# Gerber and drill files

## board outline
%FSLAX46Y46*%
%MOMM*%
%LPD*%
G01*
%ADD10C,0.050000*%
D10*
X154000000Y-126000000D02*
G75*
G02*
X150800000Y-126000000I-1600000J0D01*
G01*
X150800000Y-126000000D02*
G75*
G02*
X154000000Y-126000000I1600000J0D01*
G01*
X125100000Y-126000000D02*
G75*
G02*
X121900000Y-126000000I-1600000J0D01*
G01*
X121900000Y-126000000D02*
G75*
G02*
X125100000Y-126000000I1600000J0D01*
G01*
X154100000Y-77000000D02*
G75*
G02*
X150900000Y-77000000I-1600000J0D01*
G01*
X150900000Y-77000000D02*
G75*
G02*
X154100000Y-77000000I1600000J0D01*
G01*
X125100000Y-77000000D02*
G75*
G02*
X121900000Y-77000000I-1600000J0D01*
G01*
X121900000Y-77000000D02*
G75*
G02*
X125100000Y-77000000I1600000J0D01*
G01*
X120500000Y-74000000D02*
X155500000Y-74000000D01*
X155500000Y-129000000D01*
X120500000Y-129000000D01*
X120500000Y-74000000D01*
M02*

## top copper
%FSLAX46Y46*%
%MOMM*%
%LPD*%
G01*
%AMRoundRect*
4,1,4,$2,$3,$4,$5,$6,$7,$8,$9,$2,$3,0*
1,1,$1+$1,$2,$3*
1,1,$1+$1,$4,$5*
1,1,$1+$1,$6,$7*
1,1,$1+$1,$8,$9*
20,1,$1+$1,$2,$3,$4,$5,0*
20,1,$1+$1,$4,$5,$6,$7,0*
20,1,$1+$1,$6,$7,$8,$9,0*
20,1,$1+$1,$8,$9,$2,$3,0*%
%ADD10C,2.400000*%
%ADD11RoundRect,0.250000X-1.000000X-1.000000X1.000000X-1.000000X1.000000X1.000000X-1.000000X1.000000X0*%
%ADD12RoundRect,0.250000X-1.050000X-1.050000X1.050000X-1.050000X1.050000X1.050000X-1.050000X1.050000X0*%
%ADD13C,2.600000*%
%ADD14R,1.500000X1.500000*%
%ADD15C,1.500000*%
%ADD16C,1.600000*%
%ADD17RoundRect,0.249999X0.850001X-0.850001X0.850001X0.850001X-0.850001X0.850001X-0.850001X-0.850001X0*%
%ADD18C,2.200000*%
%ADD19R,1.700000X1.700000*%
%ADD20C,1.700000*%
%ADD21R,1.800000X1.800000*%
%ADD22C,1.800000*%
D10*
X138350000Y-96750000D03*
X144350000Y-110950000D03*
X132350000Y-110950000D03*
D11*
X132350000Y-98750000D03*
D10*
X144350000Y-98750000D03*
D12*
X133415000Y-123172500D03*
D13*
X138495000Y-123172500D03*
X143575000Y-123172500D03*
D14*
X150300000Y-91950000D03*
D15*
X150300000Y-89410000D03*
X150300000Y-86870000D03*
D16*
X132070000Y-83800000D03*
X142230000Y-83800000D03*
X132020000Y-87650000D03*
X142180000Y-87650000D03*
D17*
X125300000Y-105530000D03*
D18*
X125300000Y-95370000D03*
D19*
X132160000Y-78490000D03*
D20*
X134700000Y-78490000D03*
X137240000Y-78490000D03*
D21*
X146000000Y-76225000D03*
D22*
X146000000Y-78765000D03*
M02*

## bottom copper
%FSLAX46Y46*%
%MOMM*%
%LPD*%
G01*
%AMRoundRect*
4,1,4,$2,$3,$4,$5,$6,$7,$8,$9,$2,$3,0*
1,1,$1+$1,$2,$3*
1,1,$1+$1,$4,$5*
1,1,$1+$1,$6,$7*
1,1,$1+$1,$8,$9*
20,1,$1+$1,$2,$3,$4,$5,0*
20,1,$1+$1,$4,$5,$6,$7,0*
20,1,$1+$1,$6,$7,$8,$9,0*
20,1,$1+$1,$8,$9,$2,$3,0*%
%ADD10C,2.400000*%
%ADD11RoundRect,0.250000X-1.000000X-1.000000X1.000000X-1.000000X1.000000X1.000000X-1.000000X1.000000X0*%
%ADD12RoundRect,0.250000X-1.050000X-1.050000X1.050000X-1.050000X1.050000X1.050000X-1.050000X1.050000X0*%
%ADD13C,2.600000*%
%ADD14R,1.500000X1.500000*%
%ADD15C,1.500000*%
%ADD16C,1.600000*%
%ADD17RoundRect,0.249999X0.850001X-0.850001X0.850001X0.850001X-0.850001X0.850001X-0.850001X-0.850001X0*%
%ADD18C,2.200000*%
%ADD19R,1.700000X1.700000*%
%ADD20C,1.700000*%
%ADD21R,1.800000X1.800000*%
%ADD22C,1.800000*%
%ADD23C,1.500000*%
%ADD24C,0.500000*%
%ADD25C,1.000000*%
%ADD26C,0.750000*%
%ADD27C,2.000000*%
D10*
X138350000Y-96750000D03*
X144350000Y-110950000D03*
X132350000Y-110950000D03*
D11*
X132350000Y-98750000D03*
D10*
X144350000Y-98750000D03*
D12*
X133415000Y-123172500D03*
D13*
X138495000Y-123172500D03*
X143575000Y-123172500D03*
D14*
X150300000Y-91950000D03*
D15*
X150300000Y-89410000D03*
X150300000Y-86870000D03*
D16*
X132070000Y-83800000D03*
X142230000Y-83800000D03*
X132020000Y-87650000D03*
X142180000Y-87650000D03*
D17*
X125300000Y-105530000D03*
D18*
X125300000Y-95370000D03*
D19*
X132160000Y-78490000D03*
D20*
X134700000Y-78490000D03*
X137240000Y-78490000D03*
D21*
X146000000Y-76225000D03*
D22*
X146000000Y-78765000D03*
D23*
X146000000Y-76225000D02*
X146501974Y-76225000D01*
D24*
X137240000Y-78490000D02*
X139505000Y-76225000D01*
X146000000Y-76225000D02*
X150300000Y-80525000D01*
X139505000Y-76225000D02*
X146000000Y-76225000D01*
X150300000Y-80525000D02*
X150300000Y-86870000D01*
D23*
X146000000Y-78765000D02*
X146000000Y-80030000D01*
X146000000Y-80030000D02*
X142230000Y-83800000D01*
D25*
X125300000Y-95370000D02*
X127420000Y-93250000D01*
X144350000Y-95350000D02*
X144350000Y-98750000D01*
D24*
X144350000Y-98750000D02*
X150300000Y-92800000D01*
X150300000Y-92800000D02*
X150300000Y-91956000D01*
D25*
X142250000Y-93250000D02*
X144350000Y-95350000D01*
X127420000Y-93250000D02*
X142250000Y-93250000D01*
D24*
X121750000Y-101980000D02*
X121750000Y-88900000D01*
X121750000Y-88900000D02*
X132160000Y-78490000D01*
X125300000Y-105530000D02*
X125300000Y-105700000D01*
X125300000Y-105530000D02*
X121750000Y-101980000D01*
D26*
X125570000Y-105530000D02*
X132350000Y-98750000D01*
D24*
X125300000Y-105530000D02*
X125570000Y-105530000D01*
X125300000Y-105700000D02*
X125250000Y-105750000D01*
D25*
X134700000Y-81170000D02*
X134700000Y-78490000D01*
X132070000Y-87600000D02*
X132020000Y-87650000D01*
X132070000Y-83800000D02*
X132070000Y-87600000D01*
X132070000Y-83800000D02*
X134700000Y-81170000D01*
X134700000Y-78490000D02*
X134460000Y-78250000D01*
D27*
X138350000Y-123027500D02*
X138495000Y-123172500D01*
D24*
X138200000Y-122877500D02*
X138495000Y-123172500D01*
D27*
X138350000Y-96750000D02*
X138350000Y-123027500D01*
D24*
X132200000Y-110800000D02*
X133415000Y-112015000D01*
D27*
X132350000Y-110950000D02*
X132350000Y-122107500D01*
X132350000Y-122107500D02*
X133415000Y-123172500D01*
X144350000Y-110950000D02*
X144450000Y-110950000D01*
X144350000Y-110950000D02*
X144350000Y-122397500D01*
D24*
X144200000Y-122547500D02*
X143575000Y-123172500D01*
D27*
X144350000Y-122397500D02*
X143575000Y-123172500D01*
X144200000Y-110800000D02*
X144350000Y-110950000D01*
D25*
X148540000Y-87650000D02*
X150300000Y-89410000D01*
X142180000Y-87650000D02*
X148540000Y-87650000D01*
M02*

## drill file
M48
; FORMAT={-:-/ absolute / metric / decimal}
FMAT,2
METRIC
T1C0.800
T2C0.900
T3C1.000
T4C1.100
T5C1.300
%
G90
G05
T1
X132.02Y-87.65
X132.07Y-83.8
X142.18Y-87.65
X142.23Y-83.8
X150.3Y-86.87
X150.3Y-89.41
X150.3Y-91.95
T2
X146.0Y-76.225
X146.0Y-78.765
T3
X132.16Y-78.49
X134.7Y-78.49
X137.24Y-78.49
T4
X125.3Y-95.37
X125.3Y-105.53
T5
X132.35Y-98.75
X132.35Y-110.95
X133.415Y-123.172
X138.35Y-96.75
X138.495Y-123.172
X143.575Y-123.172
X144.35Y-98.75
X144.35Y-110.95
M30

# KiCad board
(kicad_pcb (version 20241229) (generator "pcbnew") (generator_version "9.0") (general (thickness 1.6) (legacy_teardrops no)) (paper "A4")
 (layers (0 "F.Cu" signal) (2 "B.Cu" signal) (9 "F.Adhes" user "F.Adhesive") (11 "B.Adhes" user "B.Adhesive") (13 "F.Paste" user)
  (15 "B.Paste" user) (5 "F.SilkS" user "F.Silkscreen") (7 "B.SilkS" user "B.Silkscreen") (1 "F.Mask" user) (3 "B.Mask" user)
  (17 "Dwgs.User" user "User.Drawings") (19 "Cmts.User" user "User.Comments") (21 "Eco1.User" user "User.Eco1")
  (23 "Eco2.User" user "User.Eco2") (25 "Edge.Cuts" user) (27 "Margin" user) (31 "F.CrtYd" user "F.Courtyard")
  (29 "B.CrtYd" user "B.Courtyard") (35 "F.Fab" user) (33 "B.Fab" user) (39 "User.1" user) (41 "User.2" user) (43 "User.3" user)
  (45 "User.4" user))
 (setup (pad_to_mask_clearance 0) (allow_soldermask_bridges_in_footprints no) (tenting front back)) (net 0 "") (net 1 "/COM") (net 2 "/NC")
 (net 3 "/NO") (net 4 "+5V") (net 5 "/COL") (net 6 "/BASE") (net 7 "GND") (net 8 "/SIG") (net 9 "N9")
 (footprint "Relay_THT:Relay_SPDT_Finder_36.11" (layer "F.Cu") (at 132.35 98.75)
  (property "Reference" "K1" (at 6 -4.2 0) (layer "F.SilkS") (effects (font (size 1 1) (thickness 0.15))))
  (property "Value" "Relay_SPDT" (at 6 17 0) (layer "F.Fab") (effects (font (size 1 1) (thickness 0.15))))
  (pad "11" thru_hole circle (at 6 -2) (size 2.4 2.4) (drill 1.3) (layers "*.Cu" "*.Mask") (remove_unused_layers no) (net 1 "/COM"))
  (pad "12" thru_hole circle (at 12 12.2) (size 2.4 2.4) (drill 1.3) (layers "*.Cu" "*.Mask") (remove_unused_layers no) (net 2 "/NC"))
  (pad "14" thru_hole circle (at 0 12.2) (size 2.4 2.4) (drill 1.3) (layers "*.Cu" "*.Mask") (remove_unused_layers no) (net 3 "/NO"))
  (pad "A1" thru_hole roundrect (at 0 0) (size 2.5 2.5) (drill 1.3) (layers "*.Cu" "*.Mask") (remove_unused_layers no)
   (roundrect_rratio 0.1) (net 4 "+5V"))
  (pad "A2" thru_hole circle (at 12 0) (size 2.4 2.4) (drill 1.3) (layers "*.Cu" "*.Mask") (remove_unused_layers no) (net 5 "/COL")))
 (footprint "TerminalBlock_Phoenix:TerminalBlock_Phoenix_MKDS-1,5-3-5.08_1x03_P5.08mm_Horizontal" (layer "F.Cu") (at 133.415 123.1725)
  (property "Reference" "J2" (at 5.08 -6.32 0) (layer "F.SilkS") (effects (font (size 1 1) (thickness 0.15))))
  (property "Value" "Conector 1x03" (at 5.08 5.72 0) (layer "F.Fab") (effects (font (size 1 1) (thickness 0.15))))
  (pad "1" thru_hole roundrect (at 0 0) (size 2.6 2.6) (drill 1.3) (layers "*.Cu" "*.Mask") (remove_unused_layers no)
   (roundrect_rratio 0.096154) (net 3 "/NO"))
  (pad "2" thru_hole circle (at 5.08 0) (size 2.6 2.6) (drill 1.3) (layers "*.Cu" "*.Mask") (remove_unused_layers no) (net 1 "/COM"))
  (pad "3" thru_hole circle (at 10.16 0) (size 2.6 2.6) (drill 1.3) (layers "*.Cu" "*.Mask") (remove_unused_layers no) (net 2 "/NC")))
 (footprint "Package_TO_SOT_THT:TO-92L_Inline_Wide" (layer "F.Cu") (at 150.3 91.95 90)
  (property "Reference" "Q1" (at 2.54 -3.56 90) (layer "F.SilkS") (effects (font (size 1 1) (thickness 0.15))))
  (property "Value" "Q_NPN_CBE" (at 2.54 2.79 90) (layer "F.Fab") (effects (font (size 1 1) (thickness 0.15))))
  (pad "1" thru_hole rect (at 0 0 90) (size 1.5 1.5) (drill 0.8) (layers "*.Cu" "*.Mask") (remove_unused_layers no) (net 5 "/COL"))
  (pad "2" thru_hole circle (at 2.54 0 90) (size 1.5 1.5) (drill 0.8) (layers "*.Cu" "*.Mask") (remove_unused_layers no) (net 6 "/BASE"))
  (pad "3" thru_hole circle (at 5.08 0 90) (size 1.5 1.5) (drill 0.8) (layers "*.Cu" "*.Mask") (remove_unused_layers no) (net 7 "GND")))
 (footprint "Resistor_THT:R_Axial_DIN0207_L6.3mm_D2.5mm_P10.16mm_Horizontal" (layer "F.Cu") (at 132.07 83.8)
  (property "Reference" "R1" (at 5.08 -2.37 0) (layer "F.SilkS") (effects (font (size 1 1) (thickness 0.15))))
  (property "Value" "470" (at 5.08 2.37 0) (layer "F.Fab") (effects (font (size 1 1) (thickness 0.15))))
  (pad "1" thru_hole circle (at 0 0) (size 1.6 1.6) (drill 0.8) (layers "*.Cu" "*.Mask") (remove_unused_layers no) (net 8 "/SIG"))
  (pad "2" thru_hole circle (at 10.16 0) (size 1.6 1.6) (drill 0.8) (layers "*.Cu" "*.Mask") (remove_unused_layers no) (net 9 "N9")))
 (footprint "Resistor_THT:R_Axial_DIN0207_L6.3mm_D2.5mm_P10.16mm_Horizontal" (layer "F.Cu") (at 132.02 87.65)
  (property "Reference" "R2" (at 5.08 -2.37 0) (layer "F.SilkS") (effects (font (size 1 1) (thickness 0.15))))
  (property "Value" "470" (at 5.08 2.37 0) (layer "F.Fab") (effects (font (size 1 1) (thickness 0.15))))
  (pad "1" thru_hole circle (at 0 0) (size 1.6 1.6) (drill 0.8) (layers "*.Cu" "*.Mask") (remove_unused_layers no) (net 8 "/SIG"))
  (pad "2" thru_hole circle (at 10.16 0) (size 1.6 1.6) (drill 0.8) (layers "*.Cu" "*.Mask") (remove_unused_layers no) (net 6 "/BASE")))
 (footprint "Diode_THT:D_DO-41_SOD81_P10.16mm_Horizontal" (layer "F.Cu") (at 125.3 105.53 90)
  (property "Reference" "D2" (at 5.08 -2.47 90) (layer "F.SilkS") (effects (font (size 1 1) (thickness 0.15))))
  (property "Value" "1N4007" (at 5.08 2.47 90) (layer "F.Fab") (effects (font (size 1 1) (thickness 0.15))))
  (pad "1" thru_hole roundrect (at 0 0 90) (size 2.2 2.2) (drill 1.1) (layers "*.Cu" "*.Mask") (remove_unused_layers no)
   (roundrect_rratio 0.113636) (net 4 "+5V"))
  (pad "2" thru_hole circle (at 10.16 0 90) (size 2.2 2.2) (drill 1.1) (layers "*.Cu" "*.Mask") (remove_unused_layers no) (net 5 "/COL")))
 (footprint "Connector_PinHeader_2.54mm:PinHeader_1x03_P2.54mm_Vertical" (layer "F.Cu") (at 132.16 78.49 90)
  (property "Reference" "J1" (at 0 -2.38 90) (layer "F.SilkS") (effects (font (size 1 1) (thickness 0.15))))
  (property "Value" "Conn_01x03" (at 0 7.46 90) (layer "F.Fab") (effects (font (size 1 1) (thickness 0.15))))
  (pad "1" thru_hole rect (at 0 0 90) (size 1.7 1.7) (drill 1) (layers "*.Cu" "*.Mask") (remove_unused_layers no) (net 4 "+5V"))
  (pad "2" thru_hole circle (at 0 2.54 90) (size 1.7 1.7) (drill 1) (layers "*.Cu" "*.Mask") (remove_unused_layers no) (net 8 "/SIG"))
  (pad "3" thru_hole circle (at 0 5.08 90) (size 1.7 1.7) (drill 1) (layers "*.Cu" "*.Mask") (remove_unused_layers no) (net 7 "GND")))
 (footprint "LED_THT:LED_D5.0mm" (layer "F.Cu") (at 146 76.225 -90)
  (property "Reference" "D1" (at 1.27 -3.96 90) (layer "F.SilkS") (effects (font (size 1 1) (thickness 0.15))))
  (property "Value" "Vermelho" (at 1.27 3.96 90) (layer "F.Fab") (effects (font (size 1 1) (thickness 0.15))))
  (pad "1" thru_hole rect (at 0 0 270) (size 1.8 1.8) (drill 0.9) (layers "*.Cu" "*.Mask") (remove_unused_layers no) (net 7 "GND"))
  (pad "2" thru_hole circle (at 2.54 0 270) (size 1.8 1.8) (drill 0.9) (layers "*.Cu" "*.Mask") (remove_unused_layers no) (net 9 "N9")))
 (gr_circle (center 152.4 126) (end 154 126) (stroke (width 0.05) (type solid)) (fill no) (layer "Edge.Cuts"))
 (gr_circle (center 123.5 126) (end 125.1 126) (stroke (width 0.05) (type solid)) (fill no) (layer "Edge.Cuts"))
 (gr_circle (center 152.5 77) (end 154.1 77) (stroke (width 0.05) (type solid)) (fill no) (layer "Edge.Cuts"))
 (gr_circle (center 123.5 77) (end 125.1 77) (stroke (width 0.05) (type solid)) (fill no) (layer "Edge.Cuts"))
 (gr_rect (start 120.5 74) (end 155.5 129) (stroke (width 0.05) (type default)) (fill no) (layer "Edge.Cuts"))
 (segment (start 146 76.225) (end 146.501974 76.225) (width 1.5) (layer "B.Cu") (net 7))
 (segment (start 137.24 78.49) (end 139.505 76.225) (width 0.5) (layer "B.Cu") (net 7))
 (segment (start 146 76.225) (end 150.3 80.525) (width 0.5) (layer "B.Cu") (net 7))
 (segment (start 139.505 76.225) (end 146 76.225) (width 0.5) (layer "B.Cu") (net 7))
 (segment (start 150.3 80.525) (end 150.3 86.87) (width 0.5) (layer "B.Cu") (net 7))
 (segment (start 146 78.765) (end 146 80.03) (width 1.5) (layer "B.Cu") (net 9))
 (segment (start 146 80.03) (end 142.23 83.8) (width 1.5) (layer "B.Cu") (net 9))
 (segment (start 125.3 95.37) (end 127.42 93.25) (width 1) (layer "B.Cu") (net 5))
 (segment (start 144.35 95.35) (end 144.35 98.75) (width 1) (layer "B.Cu") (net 5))
 (segment (start 144.35 98.75) (end 150.3 92.8) (width 0.5) (layer "B.Cu") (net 5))
 (segment (start 150.3 92.8) (end 150.3 91.956) (width 0.5) (layer "B.Cu") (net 5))
 (segment (start 142.25 93.25) (end 144.35 95.35) (width 1) (layer "B.Cu") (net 5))
 (segment (start 127.42 93.25) (end 142.25 93.25) (width 1) (layer "B.Cu") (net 5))
 (segment (start 121.75 101.98) (end 121.75 88.9) (width 0.5) (layer "B.Cu") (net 4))
 (segment (start 121.75 88.9) (end 132.16 78.49) (width 0.5) (layer "B.Cu") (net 4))
 (segment (start 125.3 105.53) (end 125.3 105.7) (width 0.5) (layer "B.Cu") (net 4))
 (segment (start 125.3 105.53) (end 121.75 101.98) (width 0.5) (layer "B.Cu") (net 4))
 (segment (start 125.57 105.53) (end 132.35 98.75) (width 0.75) (layer "B.Cu") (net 4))
 (segment (start 125.3 105.53) (end 125.57 105.53) (width 0.5) (layer "B.Cu") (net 4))
 (segment (start 125.3 105.7) (end 125.25 105.75) (width 0.5) (layer "B.Cu") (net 4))
 (segment (start 134.7 81.17) (end 134.7 78.49) (width 1) (layer "B.Cu") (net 8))
 (segment (start 132.07 87.6) (end 132.02 87.65) (width 1) (layer "B.Cu") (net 8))
 (segment (start 132.07 83.8) (end 132.07 87.6) (width 1) (layer "B.Cu") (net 8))
 (segment (start 132.07 83.8) (end 134.7 81.17) (width 1) (layer "B.Cu") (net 8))
 (segment (start 134.7 78.49) (end 134.46 78.25) (width 1) (layer "B.Cu") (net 8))
 (segment (start 138.35 123.0275) (end 138.495 123.1725) (width 2) (layer "B.Cu") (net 1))
 (segment (start 138.2 122.8775) (end 138.495 123.1725) (width 0.5) (layer "B.Cu") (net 1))
 (segment (start 138.35 96.75) (end 138.35 123.0275) (width 2) (layer "B.Cu") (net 1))
 (segment (start 132.2 110.8) (end 133.415 112.015) (width 0.5) (layer "B.Cu") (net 3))
 (segment (start 132.35 110.95) (end 132.35 122.1075) (width 2) (layer "B.Cu") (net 3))
 (segment (start 132.35 122.1075) (end 133.415 123.1725) (width 2) (layer "B.Cu") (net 3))
 (segment (start 144.35 110.95) (end 144.45 110.95) (width 2) (layer "B.Cu") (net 2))
 (segment (start 144.35 110.95) (end 144.35 122.3975) (width 2) (layer "B.Cu") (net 2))
 (segment (start 144.2 122.5475) (end 143.575 123.1725) (width 0.5) (layer "B.Cu") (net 2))
 (segment (start 144.35 122.3975) (end 143.575 123.1725) (width 2) (layer "B.Cu") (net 2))
 (segment (start 144.2 110.8) (end 144.35 110.95) (width 2) (layer "B.Cu") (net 2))
 (segment (start 148.54 87.65) (end 150.3 89.41) (width 1) (layer "B.Cu") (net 6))
 (segment (start 142.18 87.65) (end 148.54 87.65) (width 1) (layer "B.Cu") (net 6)))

